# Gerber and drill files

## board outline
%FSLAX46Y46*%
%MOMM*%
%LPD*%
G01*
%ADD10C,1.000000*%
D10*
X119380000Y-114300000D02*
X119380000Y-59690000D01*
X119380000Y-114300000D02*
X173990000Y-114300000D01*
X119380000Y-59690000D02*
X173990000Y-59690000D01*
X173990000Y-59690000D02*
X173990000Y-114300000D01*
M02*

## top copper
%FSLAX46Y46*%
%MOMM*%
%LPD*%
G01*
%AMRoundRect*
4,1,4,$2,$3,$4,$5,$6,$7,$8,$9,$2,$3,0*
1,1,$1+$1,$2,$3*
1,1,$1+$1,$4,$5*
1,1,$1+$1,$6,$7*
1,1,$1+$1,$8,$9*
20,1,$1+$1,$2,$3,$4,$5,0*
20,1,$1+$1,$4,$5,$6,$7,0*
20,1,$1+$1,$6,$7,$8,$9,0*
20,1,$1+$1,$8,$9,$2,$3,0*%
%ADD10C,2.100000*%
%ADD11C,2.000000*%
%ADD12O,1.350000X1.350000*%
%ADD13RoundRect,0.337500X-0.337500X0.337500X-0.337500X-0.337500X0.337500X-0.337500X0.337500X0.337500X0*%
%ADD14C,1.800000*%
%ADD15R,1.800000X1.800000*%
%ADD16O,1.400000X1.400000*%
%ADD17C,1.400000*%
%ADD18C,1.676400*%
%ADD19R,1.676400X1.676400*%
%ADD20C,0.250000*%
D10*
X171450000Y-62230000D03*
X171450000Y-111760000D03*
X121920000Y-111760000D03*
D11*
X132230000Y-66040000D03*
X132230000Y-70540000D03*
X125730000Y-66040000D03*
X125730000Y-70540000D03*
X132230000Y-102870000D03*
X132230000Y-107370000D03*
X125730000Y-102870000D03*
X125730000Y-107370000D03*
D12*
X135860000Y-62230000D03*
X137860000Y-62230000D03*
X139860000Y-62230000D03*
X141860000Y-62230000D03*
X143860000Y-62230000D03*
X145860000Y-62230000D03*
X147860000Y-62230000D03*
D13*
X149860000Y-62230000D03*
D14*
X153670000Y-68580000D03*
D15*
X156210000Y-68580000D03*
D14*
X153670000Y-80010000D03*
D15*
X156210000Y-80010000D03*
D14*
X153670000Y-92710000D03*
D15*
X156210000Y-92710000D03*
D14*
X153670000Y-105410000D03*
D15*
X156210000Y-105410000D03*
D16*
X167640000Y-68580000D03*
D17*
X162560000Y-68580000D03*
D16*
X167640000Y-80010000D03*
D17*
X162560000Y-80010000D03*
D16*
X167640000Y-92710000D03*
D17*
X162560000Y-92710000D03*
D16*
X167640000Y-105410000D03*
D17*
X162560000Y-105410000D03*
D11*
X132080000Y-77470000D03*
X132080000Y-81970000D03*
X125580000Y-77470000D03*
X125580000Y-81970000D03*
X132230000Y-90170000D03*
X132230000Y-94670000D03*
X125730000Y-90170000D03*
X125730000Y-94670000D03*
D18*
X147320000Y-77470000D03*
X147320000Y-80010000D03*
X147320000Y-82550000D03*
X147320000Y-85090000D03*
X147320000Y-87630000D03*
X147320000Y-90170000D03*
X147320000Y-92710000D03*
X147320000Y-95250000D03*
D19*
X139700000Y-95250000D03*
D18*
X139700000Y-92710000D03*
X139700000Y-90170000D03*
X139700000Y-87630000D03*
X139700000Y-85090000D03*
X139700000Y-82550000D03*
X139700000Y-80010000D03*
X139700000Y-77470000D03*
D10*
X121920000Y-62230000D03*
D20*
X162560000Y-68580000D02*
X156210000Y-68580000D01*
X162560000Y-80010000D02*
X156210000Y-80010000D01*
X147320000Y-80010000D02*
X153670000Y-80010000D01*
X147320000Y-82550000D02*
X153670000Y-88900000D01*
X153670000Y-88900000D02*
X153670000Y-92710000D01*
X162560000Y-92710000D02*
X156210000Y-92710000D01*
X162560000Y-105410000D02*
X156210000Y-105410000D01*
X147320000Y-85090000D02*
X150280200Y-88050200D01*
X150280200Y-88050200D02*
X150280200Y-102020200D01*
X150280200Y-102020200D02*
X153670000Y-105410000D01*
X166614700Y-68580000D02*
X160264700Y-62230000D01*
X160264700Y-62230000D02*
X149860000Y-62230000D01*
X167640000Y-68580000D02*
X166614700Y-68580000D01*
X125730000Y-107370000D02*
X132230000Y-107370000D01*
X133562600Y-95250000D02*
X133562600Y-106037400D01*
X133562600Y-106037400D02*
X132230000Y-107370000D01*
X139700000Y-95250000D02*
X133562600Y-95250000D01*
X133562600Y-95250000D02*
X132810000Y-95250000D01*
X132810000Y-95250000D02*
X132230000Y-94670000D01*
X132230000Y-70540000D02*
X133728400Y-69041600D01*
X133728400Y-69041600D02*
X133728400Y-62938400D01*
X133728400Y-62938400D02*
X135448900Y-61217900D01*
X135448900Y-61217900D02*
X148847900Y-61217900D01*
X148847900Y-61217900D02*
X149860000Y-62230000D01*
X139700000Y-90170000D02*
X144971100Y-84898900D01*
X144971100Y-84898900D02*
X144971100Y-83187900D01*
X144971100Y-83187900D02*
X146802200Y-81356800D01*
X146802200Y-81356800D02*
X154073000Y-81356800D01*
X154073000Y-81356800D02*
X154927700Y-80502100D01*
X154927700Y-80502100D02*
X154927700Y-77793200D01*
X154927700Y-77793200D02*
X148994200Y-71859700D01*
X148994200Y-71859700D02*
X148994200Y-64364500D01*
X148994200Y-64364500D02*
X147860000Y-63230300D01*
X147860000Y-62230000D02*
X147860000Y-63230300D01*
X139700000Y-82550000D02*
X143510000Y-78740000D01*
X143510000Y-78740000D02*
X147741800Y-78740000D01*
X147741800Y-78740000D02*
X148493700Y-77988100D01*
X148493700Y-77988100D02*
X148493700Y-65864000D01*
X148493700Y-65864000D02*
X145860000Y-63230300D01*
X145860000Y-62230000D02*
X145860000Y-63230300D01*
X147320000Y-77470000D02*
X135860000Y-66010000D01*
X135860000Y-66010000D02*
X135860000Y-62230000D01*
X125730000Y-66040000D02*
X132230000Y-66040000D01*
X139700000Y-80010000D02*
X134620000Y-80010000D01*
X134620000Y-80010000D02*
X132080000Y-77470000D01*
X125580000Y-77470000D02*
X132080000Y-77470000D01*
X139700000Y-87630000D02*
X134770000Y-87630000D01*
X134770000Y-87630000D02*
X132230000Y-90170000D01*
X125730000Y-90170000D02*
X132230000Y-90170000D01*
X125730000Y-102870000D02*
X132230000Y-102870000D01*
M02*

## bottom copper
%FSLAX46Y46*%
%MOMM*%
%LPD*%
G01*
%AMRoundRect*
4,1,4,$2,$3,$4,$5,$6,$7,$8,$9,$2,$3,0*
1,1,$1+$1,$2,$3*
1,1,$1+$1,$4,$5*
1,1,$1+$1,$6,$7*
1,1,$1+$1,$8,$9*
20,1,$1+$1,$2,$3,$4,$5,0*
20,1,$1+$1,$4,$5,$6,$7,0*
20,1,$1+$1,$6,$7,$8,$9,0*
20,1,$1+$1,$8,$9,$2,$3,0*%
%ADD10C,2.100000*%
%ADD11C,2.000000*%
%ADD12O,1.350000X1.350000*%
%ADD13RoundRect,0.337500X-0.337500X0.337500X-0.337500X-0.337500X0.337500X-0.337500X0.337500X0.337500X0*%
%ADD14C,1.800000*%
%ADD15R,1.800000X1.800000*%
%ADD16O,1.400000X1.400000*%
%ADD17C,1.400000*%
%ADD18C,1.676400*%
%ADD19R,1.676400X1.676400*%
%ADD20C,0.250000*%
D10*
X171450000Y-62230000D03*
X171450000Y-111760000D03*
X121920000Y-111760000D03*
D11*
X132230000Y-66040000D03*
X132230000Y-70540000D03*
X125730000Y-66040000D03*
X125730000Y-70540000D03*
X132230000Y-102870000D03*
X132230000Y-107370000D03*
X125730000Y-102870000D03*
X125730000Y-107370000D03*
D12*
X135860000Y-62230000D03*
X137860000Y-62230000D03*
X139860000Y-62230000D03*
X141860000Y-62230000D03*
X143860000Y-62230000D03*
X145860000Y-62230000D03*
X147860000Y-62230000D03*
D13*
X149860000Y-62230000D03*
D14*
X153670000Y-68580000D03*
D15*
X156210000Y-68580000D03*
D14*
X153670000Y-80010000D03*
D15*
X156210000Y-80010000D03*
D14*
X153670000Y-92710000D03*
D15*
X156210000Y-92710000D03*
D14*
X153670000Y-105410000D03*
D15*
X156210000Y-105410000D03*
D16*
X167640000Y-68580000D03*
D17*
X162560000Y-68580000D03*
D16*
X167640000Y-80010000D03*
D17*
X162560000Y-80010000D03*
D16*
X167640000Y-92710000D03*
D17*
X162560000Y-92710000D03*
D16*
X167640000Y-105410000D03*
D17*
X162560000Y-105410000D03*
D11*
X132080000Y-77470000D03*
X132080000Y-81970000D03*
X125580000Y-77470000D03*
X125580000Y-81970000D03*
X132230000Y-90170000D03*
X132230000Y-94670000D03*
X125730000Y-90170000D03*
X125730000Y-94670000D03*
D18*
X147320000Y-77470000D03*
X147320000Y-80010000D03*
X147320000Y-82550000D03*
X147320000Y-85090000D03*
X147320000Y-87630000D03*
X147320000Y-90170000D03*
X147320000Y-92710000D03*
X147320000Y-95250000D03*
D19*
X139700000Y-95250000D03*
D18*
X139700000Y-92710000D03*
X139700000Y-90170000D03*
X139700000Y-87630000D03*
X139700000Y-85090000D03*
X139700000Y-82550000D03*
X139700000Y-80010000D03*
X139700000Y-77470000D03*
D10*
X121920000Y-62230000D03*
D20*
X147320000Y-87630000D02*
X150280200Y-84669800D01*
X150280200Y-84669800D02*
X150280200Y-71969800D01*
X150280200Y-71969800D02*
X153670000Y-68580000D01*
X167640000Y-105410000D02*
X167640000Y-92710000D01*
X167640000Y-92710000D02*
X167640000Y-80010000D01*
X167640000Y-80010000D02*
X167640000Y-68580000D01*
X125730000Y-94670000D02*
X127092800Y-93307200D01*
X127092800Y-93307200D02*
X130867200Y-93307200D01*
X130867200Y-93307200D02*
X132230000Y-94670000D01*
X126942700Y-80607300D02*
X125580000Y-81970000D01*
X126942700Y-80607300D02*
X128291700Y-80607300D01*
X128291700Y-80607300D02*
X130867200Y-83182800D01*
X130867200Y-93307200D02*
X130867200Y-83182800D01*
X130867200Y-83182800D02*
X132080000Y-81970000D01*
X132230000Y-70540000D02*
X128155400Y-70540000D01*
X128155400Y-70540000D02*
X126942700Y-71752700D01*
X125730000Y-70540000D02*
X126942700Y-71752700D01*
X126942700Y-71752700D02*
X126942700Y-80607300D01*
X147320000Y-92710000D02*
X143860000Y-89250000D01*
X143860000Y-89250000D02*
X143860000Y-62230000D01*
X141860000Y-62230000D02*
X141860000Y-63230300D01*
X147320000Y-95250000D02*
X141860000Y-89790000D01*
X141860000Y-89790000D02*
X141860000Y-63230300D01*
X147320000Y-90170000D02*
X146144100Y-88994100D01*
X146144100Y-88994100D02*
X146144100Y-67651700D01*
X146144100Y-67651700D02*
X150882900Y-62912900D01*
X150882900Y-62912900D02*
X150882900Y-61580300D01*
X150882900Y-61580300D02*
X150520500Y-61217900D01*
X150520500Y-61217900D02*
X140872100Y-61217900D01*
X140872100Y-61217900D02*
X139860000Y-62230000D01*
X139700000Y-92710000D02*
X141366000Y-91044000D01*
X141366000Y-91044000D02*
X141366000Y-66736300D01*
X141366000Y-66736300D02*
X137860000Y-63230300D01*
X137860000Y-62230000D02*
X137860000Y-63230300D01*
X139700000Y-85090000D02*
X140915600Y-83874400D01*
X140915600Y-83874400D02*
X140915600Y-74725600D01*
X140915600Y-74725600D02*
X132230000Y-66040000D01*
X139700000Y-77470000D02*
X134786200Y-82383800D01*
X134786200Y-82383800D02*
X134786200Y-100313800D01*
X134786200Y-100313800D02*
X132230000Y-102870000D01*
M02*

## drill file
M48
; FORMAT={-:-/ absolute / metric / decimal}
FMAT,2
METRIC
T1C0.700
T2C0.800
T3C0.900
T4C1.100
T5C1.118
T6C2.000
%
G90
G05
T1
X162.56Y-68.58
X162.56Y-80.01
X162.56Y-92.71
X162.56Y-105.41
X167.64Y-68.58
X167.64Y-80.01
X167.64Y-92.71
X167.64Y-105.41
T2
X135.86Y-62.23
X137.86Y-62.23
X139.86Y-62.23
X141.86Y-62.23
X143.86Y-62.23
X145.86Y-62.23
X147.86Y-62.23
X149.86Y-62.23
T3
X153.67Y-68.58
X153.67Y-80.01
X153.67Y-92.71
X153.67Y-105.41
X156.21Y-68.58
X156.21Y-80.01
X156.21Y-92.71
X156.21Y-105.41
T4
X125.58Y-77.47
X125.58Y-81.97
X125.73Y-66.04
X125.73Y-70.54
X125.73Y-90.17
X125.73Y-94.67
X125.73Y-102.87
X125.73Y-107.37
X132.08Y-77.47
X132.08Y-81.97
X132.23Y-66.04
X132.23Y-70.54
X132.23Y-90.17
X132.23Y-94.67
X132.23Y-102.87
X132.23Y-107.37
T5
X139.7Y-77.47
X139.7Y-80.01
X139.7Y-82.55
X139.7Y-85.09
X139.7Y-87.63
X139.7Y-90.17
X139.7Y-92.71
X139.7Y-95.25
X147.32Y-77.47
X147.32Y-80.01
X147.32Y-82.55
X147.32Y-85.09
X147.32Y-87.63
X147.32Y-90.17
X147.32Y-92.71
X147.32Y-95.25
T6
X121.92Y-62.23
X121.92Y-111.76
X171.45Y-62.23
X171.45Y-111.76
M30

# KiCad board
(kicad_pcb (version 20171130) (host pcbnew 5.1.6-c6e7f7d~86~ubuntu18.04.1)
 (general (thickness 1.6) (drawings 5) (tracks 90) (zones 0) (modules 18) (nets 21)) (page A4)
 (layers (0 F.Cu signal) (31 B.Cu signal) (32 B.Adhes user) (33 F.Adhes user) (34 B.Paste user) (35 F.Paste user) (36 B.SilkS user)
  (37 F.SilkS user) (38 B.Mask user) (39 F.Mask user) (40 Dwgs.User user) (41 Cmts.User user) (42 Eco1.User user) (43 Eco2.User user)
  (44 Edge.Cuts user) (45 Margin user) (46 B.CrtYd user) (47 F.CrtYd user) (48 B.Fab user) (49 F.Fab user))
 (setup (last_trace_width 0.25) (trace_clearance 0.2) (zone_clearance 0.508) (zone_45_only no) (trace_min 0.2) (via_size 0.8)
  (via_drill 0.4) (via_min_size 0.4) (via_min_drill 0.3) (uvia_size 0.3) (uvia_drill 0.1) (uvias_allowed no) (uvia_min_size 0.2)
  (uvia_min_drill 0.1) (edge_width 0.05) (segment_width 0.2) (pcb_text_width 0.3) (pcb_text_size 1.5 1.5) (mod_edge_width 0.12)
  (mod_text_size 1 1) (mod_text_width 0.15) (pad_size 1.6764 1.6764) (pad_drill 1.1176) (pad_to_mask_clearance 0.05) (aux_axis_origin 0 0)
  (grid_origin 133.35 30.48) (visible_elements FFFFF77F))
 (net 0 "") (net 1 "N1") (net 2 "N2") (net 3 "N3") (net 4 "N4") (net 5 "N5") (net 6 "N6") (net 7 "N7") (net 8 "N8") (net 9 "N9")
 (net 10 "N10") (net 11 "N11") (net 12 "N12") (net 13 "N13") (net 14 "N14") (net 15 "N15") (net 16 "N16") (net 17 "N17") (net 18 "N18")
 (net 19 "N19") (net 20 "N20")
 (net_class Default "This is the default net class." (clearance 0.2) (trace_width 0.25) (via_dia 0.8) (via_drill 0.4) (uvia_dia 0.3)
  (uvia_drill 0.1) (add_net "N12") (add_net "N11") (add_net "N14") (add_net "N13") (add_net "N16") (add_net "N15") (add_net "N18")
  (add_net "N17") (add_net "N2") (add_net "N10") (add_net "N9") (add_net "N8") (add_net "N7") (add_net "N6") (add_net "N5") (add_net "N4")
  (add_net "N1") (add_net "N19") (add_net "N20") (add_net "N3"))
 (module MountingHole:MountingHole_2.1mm (layer F.Cu) (at 171.45 62.23)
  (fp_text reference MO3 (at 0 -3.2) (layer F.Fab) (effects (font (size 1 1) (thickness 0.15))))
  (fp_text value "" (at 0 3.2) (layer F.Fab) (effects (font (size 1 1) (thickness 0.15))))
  (pad "" np_thru_hole circle (at 0 0) (size 2.1 2.1) (drill 2) (layers *.Cu *.Mask)))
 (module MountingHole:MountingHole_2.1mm (layer F.Cu) (at 171.45 111.76)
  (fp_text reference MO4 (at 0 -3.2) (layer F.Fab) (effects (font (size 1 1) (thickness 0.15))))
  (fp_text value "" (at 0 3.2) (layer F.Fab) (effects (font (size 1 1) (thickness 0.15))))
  (pad "" np_thru_hole circle (at 0 0) (size 2.1 2.1) (drill 2) (layers *.Cu *.Mask)))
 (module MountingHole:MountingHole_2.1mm (layer F.Cu) (at 121.92 111.76)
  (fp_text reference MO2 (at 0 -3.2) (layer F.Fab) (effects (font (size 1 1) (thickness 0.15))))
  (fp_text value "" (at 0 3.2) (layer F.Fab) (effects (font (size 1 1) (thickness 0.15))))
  (pad "" np_thru_hole circle (at 0 0) (size 2.1 2.1) (drill 2) (layers *.Cu *.Mask)))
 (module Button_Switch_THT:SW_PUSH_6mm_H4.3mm (layer F.Cu) (at 125.73 66.04)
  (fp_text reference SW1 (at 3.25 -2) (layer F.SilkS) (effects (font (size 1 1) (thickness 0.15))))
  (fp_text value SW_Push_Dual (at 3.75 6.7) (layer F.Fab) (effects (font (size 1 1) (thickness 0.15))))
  (pad 1 thru_hole circle (at 6.5 0 90) (size 2 2) (drill 1.1) (layers *.Cu *.Mask) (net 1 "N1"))
  (pad 2 thru_hole circle (at 6.5 4.5 90) (size 2 2) (drill 1.1) (layers *.Cu *.Mask) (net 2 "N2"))
  (pad 1 thru_hole circle (at 0 0 90) (size 2 2) (drill 1.1) (layers *.Cu *.Mask) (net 1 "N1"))
  (pad 2 thru_hole circle (at 0 4.5 90) (size 2 2) (drill 1.1) (layers *.Cu *.Mask) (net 2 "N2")))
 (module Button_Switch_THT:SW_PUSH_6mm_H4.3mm (layer F.Cu) (at 125.73 102.87)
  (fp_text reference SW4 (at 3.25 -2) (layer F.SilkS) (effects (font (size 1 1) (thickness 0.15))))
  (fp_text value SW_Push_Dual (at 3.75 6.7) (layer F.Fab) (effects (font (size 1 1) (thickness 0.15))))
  (pad 1 thru_hole circle (at 6.5 0 90) (size 2 2) (drill 1.1) (layers *.Cu *.Mask) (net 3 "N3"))
  (pad 2 thru_hole circle (at 6.5 4.5 90) (size 2 2) (drill 1.1) (layers *.Cu *.Mask) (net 2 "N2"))
  (pad 1 thru_hole circle (at 0 0 90) (size 2 2) (drill 1.1) (layers *.Cu *.Mask) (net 3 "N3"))
  (pad 2 thru_hole circle (at 0 4.5 90) (size 2 2) (drill 1.1) (layers *.Cu *.Mask) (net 2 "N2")))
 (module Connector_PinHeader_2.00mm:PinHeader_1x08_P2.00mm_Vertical (layer F.Cu) (at 149.86 62.23 270)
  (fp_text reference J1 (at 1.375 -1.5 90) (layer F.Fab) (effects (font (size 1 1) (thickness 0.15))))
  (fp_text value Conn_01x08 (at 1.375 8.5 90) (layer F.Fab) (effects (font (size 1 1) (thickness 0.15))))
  (pad 8 thru_hole oval (at 0 14 270) (size 1.35 1.35) (drill 0.8) (layers *.Cu *.Mask) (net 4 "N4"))
  (pad 7 thru_hole oval (at 0 12 270) (size 1.35 1.35) (drill 0.8) (layers *.Cu *.Mask) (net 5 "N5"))
  (pad 6 thru_hole oval (at 0 10 270) (size 1.35 1.35) (drill 0.8) (layers *.Cu *.Mask) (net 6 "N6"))
  (pad 5 thru_hole oval (at 0 8 270) (size 1.35 1.35) (drill 0.8) (layers *.Cu *.Mask) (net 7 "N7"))
  (pad 4 thru_hole oval (at 0 6 270) (size 1.35 1.35) (drill 0.8) (layers *.Cu *.Mask) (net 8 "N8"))
  (pad 3 thru_hole oval (at 0 4 270) (size 1.35 1.35) (drill 0.8) (layers *.Cu *.Mask) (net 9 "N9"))
  (pad ~E thru_hole oval (at 0 2 270) (size 1.35 1.35) (drill 0.8) (layers *.Cu *.Mask) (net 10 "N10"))
  (pad GND thru_hole roundrect (at 0 0 270) (size 1.35 1.35) (drill 0.8) (layers *.Cu *.Mask) (roundrect_rratio 0.25) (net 2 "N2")))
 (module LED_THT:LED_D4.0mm (layer F.Cu) (at 156.21 68.58 180)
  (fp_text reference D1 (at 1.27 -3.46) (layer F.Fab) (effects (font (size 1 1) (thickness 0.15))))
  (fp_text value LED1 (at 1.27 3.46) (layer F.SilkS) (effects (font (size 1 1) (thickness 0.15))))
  (pad 2 thru_hole circle (at 2.54 0 180) (size 1.8 1.8) (drill 0.9) (layers *.Cu *.Mask) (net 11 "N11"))
  (pad 1 thru_hole rect (at 0 0 180) (size 1.8 1.8) (drill 0.9) (layers *.Cu *.Mask) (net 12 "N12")))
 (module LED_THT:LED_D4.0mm (layer F.Cu) (at 156.21 80.01 180)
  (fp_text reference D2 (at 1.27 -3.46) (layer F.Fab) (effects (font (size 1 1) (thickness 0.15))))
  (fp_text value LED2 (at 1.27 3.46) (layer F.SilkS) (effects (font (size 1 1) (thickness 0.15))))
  (pad 2 thru_hole circle (at 2.54 0 180) (size 1.8 1.8) (drill 0.9) (layers *.Cu *.Mask) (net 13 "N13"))
  (pad 1 thru_hole rect (at 0 0 180) (size 1.8 1.8) (drill 0.9) (layers *.Cu *.Mask) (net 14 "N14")))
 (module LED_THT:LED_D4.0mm (layer F.Cu) (at 156.21 92.71 180)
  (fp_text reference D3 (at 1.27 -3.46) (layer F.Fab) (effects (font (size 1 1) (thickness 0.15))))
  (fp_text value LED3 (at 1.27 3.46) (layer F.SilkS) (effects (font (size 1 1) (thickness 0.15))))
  (pad 2 thru_hole circle (at 2.54 0 180) (size 1.8 1.8) (drill 0.9) (layers *.Cu *.Mask) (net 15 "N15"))
  (pad 1 thru_hole rect (at 0 0 180) (size 1.8 1.8) (drill 0.9) (layers *.Cu *.Mask) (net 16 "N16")))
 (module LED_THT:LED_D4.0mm (layer F.Cu) (at 156.21 105.41 180)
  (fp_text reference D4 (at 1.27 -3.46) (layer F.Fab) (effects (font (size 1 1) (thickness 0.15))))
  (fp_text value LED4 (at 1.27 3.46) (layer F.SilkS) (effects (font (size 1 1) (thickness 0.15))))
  (pad 2 thru_hole circle (at 2.54 0 180) (size 1.8 1.8) (drill 0.9) (layers *.Cu *.Mask) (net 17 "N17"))
  (pad 1 thru_hole rect (at 0 0 180) (size 1.8 1.8) (drill 0.9) (layers *.Cu *.Mask) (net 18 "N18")))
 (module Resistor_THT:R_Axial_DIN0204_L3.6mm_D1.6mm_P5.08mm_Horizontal (layer F.Cu) (at 162.56 68.58)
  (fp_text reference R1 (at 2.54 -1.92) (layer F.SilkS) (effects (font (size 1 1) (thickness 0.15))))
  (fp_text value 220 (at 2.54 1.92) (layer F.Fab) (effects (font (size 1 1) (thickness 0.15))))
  (pad 2 thru_hole oval (at 5.08 0) (size 1.4 1.4) (drill 0.7) (layers *.Cu *.Mask) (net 2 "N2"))
  (pad 1 thru_hole circle (at 0 0) (size 1.4 1.4) (drill 0.7) (layers *.Cu *.Mask) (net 12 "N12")))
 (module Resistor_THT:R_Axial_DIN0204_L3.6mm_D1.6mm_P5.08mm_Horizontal (layer F.Cu) (at 162.56 80.01)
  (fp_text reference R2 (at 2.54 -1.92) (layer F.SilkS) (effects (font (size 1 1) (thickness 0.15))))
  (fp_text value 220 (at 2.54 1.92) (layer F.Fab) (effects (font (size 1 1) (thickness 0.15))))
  (pad 2 thru_hole oval (at 5.08 0) (size 1.4 1.4) (drill 0.7) (layers *.Cu *.Mask) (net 2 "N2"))
  (pad 1 thru_hole circle (at 0 0) (size 1.4 1.4) (drill 0.7) (layers *.Cu *.Mask) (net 14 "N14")))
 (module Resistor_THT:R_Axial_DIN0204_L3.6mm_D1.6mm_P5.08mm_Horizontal (layer F.Cu) (at 162.56 92.71)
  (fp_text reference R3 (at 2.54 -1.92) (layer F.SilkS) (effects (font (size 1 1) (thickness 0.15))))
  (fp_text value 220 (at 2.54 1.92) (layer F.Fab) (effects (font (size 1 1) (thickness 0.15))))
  (pad 2 thru_hole oval (at 5.08 0) (size 1.4 1.4) (drill 0.7) (layers *.Cu *.Mask) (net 2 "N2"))
  (pad 1 thru_hole circle (at 0 0) (size 1.4 1.4) (drill 0.7) (layers *.Cu *.Mask) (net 16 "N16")))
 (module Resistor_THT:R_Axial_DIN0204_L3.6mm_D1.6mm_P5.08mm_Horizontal (layer F.Cu) (at 162.56 105.41)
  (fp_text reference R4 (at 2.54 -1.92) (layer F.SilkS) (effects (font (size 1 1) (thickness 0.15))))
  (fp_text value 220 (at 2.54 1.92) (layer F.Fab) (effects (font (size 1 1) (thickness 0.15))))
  (pad 2 thru_hole oval (at 5.08 0) (size 1.4 1.4) (drill 0.7) (layers *.Cu *.Mask) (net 2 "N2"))
  (pad 1 thru_hole circle (at 0 0) (size 1.4 1.4) (drill 0.7) (layers *.Cu *.Mask) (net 18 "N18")))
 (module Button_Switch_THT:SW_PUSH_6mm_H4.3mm (layer F.Cu) (at 125.58 77.47)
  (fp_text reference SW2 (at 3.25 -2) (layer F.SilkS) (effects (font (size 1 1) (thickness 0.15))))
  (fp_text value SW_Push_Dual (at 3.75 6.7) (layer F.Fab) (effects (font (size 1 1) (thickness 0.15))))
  (pad 1 thru_hole circle (at 6.5 0 90) (size 2 2) (drill 1.1) (layers *.Cu *.Mask) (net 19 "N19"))
  (pad 2 thru_hole circle (at 6.5 4.5 90) (size 2 2) (drill 1.1) (layers *.Cu *.Mask) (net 2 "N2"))
  (pad 1 thru_hole circle (at 0 0 90) (size 2 2) (drill 1.1) (layers *.Cu *.Mask) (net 19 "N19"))
  (pad 2 thru_hole circle (at 0 4.5 90) (size 2 2) (drill 1.1) (layers *.Cu *.Mask) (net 2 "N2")))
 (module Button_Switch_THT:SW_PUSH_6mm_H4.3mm (layer F.Cu) (at 125.73 90.17)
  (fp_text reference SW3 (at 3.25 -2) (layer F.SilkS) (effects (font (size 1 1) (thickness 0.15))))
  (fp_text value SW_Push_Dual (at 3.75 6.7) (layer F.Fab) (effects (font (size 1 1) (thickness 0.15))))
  (pad 1 thru_hole circle (at 6.5 0 90) (size 2 2) (drill 1.1) (layers *.Cu *.Mask) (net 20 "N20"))
  (pad 2 thru_hole circle (at 6.5 4.5 90) (size 2 2) (drill 1.1) (layers *.Cu *.Mask) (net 2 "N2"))
  (pad 1 thru_hole circle (at 0 0 90) (size 2 2) (drill 1.1) (layers *.Cu *.Mask) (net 20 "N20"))
  (pad 2 thru_hole circle (at 0 4.5 90) (size 2 2) (drill 1.1) (layers *.Cu *.Mask) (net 2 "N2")))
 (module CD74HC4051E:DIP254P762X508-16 (layer F.Cu) (at 147.32 95.25)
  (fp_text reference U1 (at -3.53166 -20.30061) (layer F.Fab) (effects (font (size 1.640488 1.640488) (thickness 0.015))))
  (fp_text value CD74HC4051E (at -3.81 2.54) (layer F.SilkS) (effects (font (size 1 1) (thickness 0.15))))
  (pad 16 thru_hole circle (at 0 -17.78) (size 1.6764 1.6764) (drill 1.1176) (layers *.Cu *.Mask) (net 4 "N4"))
  (pad 15 thru_hole circle (at 0 -15.24) (size 1.6764 1.6764) (drill 1.1176) (layers *.Cu *.Mask) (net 13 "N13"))
  (pad 14 thru_hole circle (at 0 -12.7) (size 1.6764 1.6764) (drill 1.1176) (layers *.Cu *.Mask) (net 15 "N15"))
  (pad 13 thru_hole circle (at 0 -10.16) (size 1.6764 1.6764) (drill 1.1176) (layers *.Cu *.Mask) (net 17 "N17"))
  (pad 12 thru_hole circle (at 0 -7.62) (size 1.6764 1.6764) (drill 1.1176) (layers *.Cu *.Mask) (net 11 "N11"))
  (pad 11 thru_hole circle (at 0 -5.08) (size 1.6764 1.6764) (drill 1.1176) (layers *.Cu *.Mask) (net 6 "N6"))
  (pad 10 thru_hole circle (at 0 -2.54) (size 1.6764 1.6764) (drill 1.1176) (layers *.Cu *.Mask) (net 8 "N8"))
  (pad 9 thru_hole circle (at 0 0) (size 1.6764 1.6764) (drill 1.1176) (layers *.Cu *.Mask) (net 7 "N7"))
  (pad 8 thru_hole rect (at -7.62 0) (size 1.6764 1.6764) (drill 1.1176) (layers *.Cu *.Mask) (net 2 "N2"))
  (pad 7 thru_hole circle (at -7.62 -2.54) (size 1.6764 1.6764) (drill 1.1176) (layers *.Cu *.Mask) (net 5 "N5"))
  (pad 6 thru_hole circle (at -7.62 -5.08) (size 1.6764 1.6764) (drill 1.1176) (layers *.Cu *.Mask) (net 10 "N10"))
  (pad 5 thru_hole circle (at -7.62 -7.62) (size 1.6764 1.6764) (drill 1.1176) (layers *.Cu *.Mask) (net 20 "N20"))
  (pad 4 thru_hole circle (at -7.62 -10.16) (size 1.6764 1.6764) (drill 1.1176) (layers *.Cu *.Mask) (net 1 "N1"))
  (pad 3 thru_hole circle (at -7.62 -12.7) (size 1.6764 1.6764) (drill 1.1176) (layers *.Cu *.Mask) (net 9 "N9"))
  (pad 2 thru_hole circle (at -7.62 -15.24) (size 1.6764 1.6764) (drill 1.1176) (layers *.Cu *.Mask) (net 19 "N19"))
  (pad 1 thru_hole circle (at -7.62 -17.78) (size 1.6764 1.6764) (drill 1.1176) (layers *.Cu *.Mask) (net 3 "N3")))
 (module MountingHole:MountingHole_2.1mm (layer F.Cu) (at 121.92 62.23)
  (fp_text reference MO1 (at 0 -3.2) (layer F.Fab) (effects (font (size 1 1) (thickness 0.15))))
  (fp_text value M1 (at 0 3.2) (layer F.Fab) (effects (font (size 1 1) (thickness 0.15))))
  (pad "" np_thru_hole circle (at 0 0) (size 2.1 2.1) (drill 2) (layers *.Cu *.Mask)))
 (gr_line (start 119.38 114.3) (end 119.38 59.69) (angle 90) (layer Edge.Cuts) (width 1))
 (gr_line (start 119.38 114.3) (end 173.99 114.3) (angle 90) (layer Edge.Cuts) (width 1))
 (gr_line (start 119.38 59.69) (end 173.99 59.69) (angle 90) (layer Edge.Cuts) (width 1))
 (gr_line (start 173.99 59.69) (end 173.99 114.3) (angle 90) (layer Edge.Cuts) (width 1))
 (segment (start 147.32 87.63) (end 150.2802 84.6698) (width 0.25) (layer B.Cu) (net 11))
 (segment (start 150.2802 84.6698) (end 150.2802 71.9698) (width 0.25) (layer B.Cu) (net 11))
 (segment (start 150.2802 71.9698) (end 153.67 68.58) (width 0.25) (layer B.Cu) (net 11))
 (segment (start 162.56 68.58) (end 156.21 68.58) (width 0.25) (layer F.Cu) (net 12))
 (segment (start 162.56 80.01) (end 156.21 80.01) (width 0.25) (layer F.Cu) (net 14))
 (segment (start 147.32 80.01) (end 153.67 80.01) (width 0.25) (layer F.Cu) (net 13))
 (segment (start 147.32 82.55) (end 153.67 88.9) (width 0.25) (layer F.Cu) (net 15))
 (segment (start 153.67 88.9) (end 153.67 92.71) (width 0.25) (layer F.Cu) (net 15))
 (segment (start 162.56 92.71) (end 156.21 92.71) (width 0.25) (layer F.Cu) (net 16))
 (segment (start 162.56 105.41) (end 156.21 105.41) (width 0.25) (layer F.Cu) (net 18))
 (segment (start 147.32 85.09) (end 150.2802 88.0502) (width 0.25) (layer F.Cu) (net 17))
 (segment (start 150.2802 88.0502) (end 150.2802 102.0202) (width 0.25) (layer F.Cu) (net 17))
 (segment (start 150.2802 102.0202) (end 153.67 105.41) (width 0.25) (layer F.Cu) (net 17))
 (segment (start 167.64 105.41) (end 167.64 92.71) (width 0.25) (layer B.Cu) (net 2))
 (segment (start 167.64 92.71) (end 167.64 80.01) (width 0.25) (layer B.Cu) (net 2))
 (segment (start 167.64 80.01) (end 167.64 68.58) (width 0.25) (layer B.Cu) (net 2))
 (segment (start 166.6147 68.58) (end 160.2647 62.23) (width 0.25) (layer F.Cu) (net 2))
 (segment (start 160.2647 62.23) (end 149.86 62.23) (width 0.25) (layer F.Cu) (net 2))
 (segment (start 167.64 68.58) (end 166.6147 68.58) (width 0.25) (layer F.Cu) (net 2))
 (segment (start 125.73 107.37) (end 132.23 107.37) (width 0.25) (layer F.Cu) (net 2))
 (segment (start 133.5626 95.25) (end 133.5626 106.0374) (width 0.25) (layer F.Cu) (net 2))
 (segment (start 133.5626 106.0374) (end 132.23 107.37) (width 0.25) (layer F.Cu) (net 2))
 (segment (start 139.7 95.25) (end 133.5626 95.25) (width 0.25) (layer F.Cu) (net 2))
 (segment (start 133.5626 95.25) (end 132.81 95.25) (width 0.25) (layer F.Cu) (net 2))
 (segment (start 132.81 95.25) (end 132.23 94.67) (width 0.25) (layer F.Cu) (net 2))
 (segment (start 132.23 70.54) (end 133.7284 69.0416) (width 0.25) (layer F.Cu) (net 2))
 (segment (start 133.7284 69.0416) (end 133.7284 62.9384) (width 0.25) (layer F.Cu) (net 2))
 (segment (start 133.7284 62.9384) (end 135.4489 61.2179) (width 0.25) (layer F.Cu) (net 2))
 (segment (start 135.4489 61.2179) (end 148.8479 61.2179) (width 0.25) (layer F.Cu) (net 2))
 (segment (start 148.8479 61.2179) (end 149.86 62.23) (width 0.25) (layer F.Cu) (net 2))
 (segment (start 125.73 94.67) (end 127.0928 93.3072) (width 0.25) (layer B.Cu) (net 2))
 (segment (start 127.0928 93.3072) (end 130.8672 93.3072) (width 0.25) (layer B.Cu) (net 2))
 (segment (start 130.8672 93.3072) (end 132.23 94.67) (width 0.25) (layer B.Cu) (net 2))
 (segment (start 126.9427 80.6073) (end 125.58 81.97) (width 0.25) (layer B.Cu) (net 2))
 (segment (start 126.9427 80.6073) (end 128.2917 80.6073) (width 0.25) (layer B.Cu) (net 2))
 (segment (start 128.2917 80.6073) (end 130.8672 83.1828) (width 0.25) (layer B.Cu) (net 2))
 (segment (start 130.8672 93.3072) (end 130.8672 83.1828) (width 0.25) (layer B.Cu) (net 2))
 (segment (start 130.8672 83.1828) (end 132.08 81.97) (width 0.25) (layer B.Cu) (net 2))
 (segment (start 132.23 70.54) (end 128.1554 70.54) (width 0.25) (layer B.Cu) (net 2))
 (segment (start 128.1554 70.54) (end 126.9427 71.7527) (width 0.25) (layer B.Cu) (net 2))
 (segment (start 125.73 70.54) (end 126.9427 71.7527) (width 0.25) (layer B.Cu) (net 2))
 (segment (start 126.9427 71.7527) (end 126.9427 80.6073) (width 0.25) (layer B.Cu) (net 2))
 (segment (start 139.7 90.17) (end 144.9711 84.8989) (width 0.25) (layer F.Cu) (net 10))
 (segment (start 144.9711 84.8989) (end 144.9711 83.1879) (width 0.25) (layer F.Cu) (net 10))
 (segment (start 144.9711 83.1879) (end 146.8022 81.3568) (width 0.25) (layer F.Cu) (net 10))
 (segment (start 146.8022 81.3568) (end 154.073 81.3568) (width 0.25) (layer F.Cu) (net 10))
 (segment (start 154.073 81.3568) (end 154.9277 80.5021) (width 0.25) (layer F.Cu) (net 10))
 (segment (start 154.9277 80.5021) (end 154.9277 77.7932) (width 0.25) (layer F.Cu) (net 10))
 (segment (start 154.9277 77.7932) (end 148.9942 71.8597) (width 0.25) (layer F.Cu) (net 10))
 (segment (start 148.9942 71.8597) (end 148.9942 64.3645) (width 0.25) (layer F.Cu) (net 10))
 (segment (start 148.9942 64.3645) (end 147.86 63.2303) (width 0.25) (layer F.Cu) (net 10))
 (segment (start 147.86 62.23) (end 147.86 63.2303) (width 0.25) (layer F.Cu) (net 10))
 (segment (start 139.7 82.55) (end 143.51 78.74) (width 0.25) (layer F.Cu) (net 9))
 (segment (start 143.51 78.74) (end 147.7418 78.74) (width 0.25) (layer F.Cu) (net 9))
 (segment (start 147.7418 78.74) (end 148.4937 77.9881) (width 0.25) (layer F.Cu) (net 9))
 (segment (start 148.4937 77.9881) (end 148.4937 65.864) (width 0.25) (layer F.Cu) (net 9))
 (segment (start 148.4937 65.864) (end 145.86 63.2303) (width 0.25) (layer F.Cu) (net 9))
 (segment (start 145.86 62.23) (end 145.86 63.2303) (width 0.25) (layer F.Cu) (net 9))
 (segment (start 147.32 92.71) (end 143.86 89.25) (width 0.25) (layer B.Cu) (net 8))
 (segment (start 143.86 89.25) (end 143.86 62.23) (width 0.25) (layer B.Cu) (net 8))
 (segment (start 141.86 62.23) (end 141.86 63.2303) (width 0.25) (layer B.Cu) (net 7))
 (segment (start 147.32 95.25) (end 141.86 89.79) (width 0.25) (layer B.Cu) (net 7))
 (segment (start 141.86 89.79) (end 141.86 63.2303) (width 0.25) (layer B.Cu) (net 7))
 (segment (start 147.32 90.17) (end 146.1441 88.9941) (width 0.25) (layer B.Cu) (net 6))
 (segment (start 146.1441 88.9941) (end 146.1441 67.6517) (width 0.25) (layer B.Cu) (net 6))
 (segment (start 146.1441 67.6517) (end 150.8829 62.9129) (width 0.25) (layer B.Cu) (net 6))
 (segment (start 150.8829 62.9129) (end 150.8829 61.5803) (width 0.25) (layer B.Cu) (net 6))
 (segment (start 150.8829 61.5803) (end 150.5205 61.2179) (width 0.25) (layer B.Cu) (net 6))
 (segment (start 150.5205 61.2179) (end 140.8721 61.2179) (width 0.25) (layer B.Cu) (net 6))
 (segment (start 140.8721 61.2179) (end 139.86 62.23) (width 0.25) (layer B.Cu) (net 6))
 (segment (start 139.7 92.71) (end 141.366 91.044) (width 0.25) (layer B.Cu) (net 5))
 (segment (start 141.366 91.044) (end 141.366 66.7363) (width 0.25) (layer B.Cu) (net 5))
 (segment (start 141.366 66.7363) (end 137.86 63.2303) (width 0.25) (layer B.Cu) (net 5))
 (segment (start 137.86 62.23) (end 137.86 63.2303) (width 0.25) (layer B.Cu) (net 5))
 (segment (start 147.32 77.47) (end 135.86 66.01) (width 0.25) (layer F.Cu) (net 4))
 (segment (start 135.86 66.01) (end 135.86 62.23) (width 0.25) (layer F.Cu) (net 4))
 (segment (start 125.73 66.04) (end 132.23 66.04) (width 0.25) (layer F.Cu) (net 1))
 (segment (start 139.7 85.09) (end 140.9156 83.8744) (width 0.25) (layer B.Cu) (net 1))
 (segment (start 140.9156 83.8744) (end 140.9156 74.7256) (width 0.25) (layer B.Cu) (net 1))
 (segment (start 140.9156 74.7256) (end 132.23 66.04) (width 0.25) (layer B.Cu) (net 1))
 (segment (start 139.7 80.01) (end 134.62 80.01) (width 0.25) (layer F.Cu) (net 19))
 (segment (start 134.62 80.01) (end 132.08 77.47) (width 0.25) (layer F.Cu) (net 19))
 (segment (start 125.58 77.47) (end 132.08 77.47) (width 0.25) (layer F.Cu) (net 19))
 (segment (start 139.7 87.63) (end 134.77 87.63) (width 0.25) (layer F.Cu) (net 20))
 (segment (start 134.77 87.63) (end 132.23 90.17) (width 0.25) (layer F.Cu) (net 20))
 (segment (start 125.73 90.17) (end 132.23 90.17) (width 0.25) (layer F.Cu) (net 20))
 (segment (start 125.73 102.87) (end 132.23 102.87) (width 0.25) (layer F.Cu) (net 3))
 (segment (start 139.7 77.47) (end 134.7862 82.3838) (width 0.25) (layer B.Cu) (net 3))
 (segment (start 134.7862 82.3838) (end 134.7862 100.3138) (width 0.25) (layer B.Cu) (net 3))
 (segment (start 134.7862 100.3138) (end 132.23 102.87) (width 0.25) (layer B.Cu) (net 3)))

